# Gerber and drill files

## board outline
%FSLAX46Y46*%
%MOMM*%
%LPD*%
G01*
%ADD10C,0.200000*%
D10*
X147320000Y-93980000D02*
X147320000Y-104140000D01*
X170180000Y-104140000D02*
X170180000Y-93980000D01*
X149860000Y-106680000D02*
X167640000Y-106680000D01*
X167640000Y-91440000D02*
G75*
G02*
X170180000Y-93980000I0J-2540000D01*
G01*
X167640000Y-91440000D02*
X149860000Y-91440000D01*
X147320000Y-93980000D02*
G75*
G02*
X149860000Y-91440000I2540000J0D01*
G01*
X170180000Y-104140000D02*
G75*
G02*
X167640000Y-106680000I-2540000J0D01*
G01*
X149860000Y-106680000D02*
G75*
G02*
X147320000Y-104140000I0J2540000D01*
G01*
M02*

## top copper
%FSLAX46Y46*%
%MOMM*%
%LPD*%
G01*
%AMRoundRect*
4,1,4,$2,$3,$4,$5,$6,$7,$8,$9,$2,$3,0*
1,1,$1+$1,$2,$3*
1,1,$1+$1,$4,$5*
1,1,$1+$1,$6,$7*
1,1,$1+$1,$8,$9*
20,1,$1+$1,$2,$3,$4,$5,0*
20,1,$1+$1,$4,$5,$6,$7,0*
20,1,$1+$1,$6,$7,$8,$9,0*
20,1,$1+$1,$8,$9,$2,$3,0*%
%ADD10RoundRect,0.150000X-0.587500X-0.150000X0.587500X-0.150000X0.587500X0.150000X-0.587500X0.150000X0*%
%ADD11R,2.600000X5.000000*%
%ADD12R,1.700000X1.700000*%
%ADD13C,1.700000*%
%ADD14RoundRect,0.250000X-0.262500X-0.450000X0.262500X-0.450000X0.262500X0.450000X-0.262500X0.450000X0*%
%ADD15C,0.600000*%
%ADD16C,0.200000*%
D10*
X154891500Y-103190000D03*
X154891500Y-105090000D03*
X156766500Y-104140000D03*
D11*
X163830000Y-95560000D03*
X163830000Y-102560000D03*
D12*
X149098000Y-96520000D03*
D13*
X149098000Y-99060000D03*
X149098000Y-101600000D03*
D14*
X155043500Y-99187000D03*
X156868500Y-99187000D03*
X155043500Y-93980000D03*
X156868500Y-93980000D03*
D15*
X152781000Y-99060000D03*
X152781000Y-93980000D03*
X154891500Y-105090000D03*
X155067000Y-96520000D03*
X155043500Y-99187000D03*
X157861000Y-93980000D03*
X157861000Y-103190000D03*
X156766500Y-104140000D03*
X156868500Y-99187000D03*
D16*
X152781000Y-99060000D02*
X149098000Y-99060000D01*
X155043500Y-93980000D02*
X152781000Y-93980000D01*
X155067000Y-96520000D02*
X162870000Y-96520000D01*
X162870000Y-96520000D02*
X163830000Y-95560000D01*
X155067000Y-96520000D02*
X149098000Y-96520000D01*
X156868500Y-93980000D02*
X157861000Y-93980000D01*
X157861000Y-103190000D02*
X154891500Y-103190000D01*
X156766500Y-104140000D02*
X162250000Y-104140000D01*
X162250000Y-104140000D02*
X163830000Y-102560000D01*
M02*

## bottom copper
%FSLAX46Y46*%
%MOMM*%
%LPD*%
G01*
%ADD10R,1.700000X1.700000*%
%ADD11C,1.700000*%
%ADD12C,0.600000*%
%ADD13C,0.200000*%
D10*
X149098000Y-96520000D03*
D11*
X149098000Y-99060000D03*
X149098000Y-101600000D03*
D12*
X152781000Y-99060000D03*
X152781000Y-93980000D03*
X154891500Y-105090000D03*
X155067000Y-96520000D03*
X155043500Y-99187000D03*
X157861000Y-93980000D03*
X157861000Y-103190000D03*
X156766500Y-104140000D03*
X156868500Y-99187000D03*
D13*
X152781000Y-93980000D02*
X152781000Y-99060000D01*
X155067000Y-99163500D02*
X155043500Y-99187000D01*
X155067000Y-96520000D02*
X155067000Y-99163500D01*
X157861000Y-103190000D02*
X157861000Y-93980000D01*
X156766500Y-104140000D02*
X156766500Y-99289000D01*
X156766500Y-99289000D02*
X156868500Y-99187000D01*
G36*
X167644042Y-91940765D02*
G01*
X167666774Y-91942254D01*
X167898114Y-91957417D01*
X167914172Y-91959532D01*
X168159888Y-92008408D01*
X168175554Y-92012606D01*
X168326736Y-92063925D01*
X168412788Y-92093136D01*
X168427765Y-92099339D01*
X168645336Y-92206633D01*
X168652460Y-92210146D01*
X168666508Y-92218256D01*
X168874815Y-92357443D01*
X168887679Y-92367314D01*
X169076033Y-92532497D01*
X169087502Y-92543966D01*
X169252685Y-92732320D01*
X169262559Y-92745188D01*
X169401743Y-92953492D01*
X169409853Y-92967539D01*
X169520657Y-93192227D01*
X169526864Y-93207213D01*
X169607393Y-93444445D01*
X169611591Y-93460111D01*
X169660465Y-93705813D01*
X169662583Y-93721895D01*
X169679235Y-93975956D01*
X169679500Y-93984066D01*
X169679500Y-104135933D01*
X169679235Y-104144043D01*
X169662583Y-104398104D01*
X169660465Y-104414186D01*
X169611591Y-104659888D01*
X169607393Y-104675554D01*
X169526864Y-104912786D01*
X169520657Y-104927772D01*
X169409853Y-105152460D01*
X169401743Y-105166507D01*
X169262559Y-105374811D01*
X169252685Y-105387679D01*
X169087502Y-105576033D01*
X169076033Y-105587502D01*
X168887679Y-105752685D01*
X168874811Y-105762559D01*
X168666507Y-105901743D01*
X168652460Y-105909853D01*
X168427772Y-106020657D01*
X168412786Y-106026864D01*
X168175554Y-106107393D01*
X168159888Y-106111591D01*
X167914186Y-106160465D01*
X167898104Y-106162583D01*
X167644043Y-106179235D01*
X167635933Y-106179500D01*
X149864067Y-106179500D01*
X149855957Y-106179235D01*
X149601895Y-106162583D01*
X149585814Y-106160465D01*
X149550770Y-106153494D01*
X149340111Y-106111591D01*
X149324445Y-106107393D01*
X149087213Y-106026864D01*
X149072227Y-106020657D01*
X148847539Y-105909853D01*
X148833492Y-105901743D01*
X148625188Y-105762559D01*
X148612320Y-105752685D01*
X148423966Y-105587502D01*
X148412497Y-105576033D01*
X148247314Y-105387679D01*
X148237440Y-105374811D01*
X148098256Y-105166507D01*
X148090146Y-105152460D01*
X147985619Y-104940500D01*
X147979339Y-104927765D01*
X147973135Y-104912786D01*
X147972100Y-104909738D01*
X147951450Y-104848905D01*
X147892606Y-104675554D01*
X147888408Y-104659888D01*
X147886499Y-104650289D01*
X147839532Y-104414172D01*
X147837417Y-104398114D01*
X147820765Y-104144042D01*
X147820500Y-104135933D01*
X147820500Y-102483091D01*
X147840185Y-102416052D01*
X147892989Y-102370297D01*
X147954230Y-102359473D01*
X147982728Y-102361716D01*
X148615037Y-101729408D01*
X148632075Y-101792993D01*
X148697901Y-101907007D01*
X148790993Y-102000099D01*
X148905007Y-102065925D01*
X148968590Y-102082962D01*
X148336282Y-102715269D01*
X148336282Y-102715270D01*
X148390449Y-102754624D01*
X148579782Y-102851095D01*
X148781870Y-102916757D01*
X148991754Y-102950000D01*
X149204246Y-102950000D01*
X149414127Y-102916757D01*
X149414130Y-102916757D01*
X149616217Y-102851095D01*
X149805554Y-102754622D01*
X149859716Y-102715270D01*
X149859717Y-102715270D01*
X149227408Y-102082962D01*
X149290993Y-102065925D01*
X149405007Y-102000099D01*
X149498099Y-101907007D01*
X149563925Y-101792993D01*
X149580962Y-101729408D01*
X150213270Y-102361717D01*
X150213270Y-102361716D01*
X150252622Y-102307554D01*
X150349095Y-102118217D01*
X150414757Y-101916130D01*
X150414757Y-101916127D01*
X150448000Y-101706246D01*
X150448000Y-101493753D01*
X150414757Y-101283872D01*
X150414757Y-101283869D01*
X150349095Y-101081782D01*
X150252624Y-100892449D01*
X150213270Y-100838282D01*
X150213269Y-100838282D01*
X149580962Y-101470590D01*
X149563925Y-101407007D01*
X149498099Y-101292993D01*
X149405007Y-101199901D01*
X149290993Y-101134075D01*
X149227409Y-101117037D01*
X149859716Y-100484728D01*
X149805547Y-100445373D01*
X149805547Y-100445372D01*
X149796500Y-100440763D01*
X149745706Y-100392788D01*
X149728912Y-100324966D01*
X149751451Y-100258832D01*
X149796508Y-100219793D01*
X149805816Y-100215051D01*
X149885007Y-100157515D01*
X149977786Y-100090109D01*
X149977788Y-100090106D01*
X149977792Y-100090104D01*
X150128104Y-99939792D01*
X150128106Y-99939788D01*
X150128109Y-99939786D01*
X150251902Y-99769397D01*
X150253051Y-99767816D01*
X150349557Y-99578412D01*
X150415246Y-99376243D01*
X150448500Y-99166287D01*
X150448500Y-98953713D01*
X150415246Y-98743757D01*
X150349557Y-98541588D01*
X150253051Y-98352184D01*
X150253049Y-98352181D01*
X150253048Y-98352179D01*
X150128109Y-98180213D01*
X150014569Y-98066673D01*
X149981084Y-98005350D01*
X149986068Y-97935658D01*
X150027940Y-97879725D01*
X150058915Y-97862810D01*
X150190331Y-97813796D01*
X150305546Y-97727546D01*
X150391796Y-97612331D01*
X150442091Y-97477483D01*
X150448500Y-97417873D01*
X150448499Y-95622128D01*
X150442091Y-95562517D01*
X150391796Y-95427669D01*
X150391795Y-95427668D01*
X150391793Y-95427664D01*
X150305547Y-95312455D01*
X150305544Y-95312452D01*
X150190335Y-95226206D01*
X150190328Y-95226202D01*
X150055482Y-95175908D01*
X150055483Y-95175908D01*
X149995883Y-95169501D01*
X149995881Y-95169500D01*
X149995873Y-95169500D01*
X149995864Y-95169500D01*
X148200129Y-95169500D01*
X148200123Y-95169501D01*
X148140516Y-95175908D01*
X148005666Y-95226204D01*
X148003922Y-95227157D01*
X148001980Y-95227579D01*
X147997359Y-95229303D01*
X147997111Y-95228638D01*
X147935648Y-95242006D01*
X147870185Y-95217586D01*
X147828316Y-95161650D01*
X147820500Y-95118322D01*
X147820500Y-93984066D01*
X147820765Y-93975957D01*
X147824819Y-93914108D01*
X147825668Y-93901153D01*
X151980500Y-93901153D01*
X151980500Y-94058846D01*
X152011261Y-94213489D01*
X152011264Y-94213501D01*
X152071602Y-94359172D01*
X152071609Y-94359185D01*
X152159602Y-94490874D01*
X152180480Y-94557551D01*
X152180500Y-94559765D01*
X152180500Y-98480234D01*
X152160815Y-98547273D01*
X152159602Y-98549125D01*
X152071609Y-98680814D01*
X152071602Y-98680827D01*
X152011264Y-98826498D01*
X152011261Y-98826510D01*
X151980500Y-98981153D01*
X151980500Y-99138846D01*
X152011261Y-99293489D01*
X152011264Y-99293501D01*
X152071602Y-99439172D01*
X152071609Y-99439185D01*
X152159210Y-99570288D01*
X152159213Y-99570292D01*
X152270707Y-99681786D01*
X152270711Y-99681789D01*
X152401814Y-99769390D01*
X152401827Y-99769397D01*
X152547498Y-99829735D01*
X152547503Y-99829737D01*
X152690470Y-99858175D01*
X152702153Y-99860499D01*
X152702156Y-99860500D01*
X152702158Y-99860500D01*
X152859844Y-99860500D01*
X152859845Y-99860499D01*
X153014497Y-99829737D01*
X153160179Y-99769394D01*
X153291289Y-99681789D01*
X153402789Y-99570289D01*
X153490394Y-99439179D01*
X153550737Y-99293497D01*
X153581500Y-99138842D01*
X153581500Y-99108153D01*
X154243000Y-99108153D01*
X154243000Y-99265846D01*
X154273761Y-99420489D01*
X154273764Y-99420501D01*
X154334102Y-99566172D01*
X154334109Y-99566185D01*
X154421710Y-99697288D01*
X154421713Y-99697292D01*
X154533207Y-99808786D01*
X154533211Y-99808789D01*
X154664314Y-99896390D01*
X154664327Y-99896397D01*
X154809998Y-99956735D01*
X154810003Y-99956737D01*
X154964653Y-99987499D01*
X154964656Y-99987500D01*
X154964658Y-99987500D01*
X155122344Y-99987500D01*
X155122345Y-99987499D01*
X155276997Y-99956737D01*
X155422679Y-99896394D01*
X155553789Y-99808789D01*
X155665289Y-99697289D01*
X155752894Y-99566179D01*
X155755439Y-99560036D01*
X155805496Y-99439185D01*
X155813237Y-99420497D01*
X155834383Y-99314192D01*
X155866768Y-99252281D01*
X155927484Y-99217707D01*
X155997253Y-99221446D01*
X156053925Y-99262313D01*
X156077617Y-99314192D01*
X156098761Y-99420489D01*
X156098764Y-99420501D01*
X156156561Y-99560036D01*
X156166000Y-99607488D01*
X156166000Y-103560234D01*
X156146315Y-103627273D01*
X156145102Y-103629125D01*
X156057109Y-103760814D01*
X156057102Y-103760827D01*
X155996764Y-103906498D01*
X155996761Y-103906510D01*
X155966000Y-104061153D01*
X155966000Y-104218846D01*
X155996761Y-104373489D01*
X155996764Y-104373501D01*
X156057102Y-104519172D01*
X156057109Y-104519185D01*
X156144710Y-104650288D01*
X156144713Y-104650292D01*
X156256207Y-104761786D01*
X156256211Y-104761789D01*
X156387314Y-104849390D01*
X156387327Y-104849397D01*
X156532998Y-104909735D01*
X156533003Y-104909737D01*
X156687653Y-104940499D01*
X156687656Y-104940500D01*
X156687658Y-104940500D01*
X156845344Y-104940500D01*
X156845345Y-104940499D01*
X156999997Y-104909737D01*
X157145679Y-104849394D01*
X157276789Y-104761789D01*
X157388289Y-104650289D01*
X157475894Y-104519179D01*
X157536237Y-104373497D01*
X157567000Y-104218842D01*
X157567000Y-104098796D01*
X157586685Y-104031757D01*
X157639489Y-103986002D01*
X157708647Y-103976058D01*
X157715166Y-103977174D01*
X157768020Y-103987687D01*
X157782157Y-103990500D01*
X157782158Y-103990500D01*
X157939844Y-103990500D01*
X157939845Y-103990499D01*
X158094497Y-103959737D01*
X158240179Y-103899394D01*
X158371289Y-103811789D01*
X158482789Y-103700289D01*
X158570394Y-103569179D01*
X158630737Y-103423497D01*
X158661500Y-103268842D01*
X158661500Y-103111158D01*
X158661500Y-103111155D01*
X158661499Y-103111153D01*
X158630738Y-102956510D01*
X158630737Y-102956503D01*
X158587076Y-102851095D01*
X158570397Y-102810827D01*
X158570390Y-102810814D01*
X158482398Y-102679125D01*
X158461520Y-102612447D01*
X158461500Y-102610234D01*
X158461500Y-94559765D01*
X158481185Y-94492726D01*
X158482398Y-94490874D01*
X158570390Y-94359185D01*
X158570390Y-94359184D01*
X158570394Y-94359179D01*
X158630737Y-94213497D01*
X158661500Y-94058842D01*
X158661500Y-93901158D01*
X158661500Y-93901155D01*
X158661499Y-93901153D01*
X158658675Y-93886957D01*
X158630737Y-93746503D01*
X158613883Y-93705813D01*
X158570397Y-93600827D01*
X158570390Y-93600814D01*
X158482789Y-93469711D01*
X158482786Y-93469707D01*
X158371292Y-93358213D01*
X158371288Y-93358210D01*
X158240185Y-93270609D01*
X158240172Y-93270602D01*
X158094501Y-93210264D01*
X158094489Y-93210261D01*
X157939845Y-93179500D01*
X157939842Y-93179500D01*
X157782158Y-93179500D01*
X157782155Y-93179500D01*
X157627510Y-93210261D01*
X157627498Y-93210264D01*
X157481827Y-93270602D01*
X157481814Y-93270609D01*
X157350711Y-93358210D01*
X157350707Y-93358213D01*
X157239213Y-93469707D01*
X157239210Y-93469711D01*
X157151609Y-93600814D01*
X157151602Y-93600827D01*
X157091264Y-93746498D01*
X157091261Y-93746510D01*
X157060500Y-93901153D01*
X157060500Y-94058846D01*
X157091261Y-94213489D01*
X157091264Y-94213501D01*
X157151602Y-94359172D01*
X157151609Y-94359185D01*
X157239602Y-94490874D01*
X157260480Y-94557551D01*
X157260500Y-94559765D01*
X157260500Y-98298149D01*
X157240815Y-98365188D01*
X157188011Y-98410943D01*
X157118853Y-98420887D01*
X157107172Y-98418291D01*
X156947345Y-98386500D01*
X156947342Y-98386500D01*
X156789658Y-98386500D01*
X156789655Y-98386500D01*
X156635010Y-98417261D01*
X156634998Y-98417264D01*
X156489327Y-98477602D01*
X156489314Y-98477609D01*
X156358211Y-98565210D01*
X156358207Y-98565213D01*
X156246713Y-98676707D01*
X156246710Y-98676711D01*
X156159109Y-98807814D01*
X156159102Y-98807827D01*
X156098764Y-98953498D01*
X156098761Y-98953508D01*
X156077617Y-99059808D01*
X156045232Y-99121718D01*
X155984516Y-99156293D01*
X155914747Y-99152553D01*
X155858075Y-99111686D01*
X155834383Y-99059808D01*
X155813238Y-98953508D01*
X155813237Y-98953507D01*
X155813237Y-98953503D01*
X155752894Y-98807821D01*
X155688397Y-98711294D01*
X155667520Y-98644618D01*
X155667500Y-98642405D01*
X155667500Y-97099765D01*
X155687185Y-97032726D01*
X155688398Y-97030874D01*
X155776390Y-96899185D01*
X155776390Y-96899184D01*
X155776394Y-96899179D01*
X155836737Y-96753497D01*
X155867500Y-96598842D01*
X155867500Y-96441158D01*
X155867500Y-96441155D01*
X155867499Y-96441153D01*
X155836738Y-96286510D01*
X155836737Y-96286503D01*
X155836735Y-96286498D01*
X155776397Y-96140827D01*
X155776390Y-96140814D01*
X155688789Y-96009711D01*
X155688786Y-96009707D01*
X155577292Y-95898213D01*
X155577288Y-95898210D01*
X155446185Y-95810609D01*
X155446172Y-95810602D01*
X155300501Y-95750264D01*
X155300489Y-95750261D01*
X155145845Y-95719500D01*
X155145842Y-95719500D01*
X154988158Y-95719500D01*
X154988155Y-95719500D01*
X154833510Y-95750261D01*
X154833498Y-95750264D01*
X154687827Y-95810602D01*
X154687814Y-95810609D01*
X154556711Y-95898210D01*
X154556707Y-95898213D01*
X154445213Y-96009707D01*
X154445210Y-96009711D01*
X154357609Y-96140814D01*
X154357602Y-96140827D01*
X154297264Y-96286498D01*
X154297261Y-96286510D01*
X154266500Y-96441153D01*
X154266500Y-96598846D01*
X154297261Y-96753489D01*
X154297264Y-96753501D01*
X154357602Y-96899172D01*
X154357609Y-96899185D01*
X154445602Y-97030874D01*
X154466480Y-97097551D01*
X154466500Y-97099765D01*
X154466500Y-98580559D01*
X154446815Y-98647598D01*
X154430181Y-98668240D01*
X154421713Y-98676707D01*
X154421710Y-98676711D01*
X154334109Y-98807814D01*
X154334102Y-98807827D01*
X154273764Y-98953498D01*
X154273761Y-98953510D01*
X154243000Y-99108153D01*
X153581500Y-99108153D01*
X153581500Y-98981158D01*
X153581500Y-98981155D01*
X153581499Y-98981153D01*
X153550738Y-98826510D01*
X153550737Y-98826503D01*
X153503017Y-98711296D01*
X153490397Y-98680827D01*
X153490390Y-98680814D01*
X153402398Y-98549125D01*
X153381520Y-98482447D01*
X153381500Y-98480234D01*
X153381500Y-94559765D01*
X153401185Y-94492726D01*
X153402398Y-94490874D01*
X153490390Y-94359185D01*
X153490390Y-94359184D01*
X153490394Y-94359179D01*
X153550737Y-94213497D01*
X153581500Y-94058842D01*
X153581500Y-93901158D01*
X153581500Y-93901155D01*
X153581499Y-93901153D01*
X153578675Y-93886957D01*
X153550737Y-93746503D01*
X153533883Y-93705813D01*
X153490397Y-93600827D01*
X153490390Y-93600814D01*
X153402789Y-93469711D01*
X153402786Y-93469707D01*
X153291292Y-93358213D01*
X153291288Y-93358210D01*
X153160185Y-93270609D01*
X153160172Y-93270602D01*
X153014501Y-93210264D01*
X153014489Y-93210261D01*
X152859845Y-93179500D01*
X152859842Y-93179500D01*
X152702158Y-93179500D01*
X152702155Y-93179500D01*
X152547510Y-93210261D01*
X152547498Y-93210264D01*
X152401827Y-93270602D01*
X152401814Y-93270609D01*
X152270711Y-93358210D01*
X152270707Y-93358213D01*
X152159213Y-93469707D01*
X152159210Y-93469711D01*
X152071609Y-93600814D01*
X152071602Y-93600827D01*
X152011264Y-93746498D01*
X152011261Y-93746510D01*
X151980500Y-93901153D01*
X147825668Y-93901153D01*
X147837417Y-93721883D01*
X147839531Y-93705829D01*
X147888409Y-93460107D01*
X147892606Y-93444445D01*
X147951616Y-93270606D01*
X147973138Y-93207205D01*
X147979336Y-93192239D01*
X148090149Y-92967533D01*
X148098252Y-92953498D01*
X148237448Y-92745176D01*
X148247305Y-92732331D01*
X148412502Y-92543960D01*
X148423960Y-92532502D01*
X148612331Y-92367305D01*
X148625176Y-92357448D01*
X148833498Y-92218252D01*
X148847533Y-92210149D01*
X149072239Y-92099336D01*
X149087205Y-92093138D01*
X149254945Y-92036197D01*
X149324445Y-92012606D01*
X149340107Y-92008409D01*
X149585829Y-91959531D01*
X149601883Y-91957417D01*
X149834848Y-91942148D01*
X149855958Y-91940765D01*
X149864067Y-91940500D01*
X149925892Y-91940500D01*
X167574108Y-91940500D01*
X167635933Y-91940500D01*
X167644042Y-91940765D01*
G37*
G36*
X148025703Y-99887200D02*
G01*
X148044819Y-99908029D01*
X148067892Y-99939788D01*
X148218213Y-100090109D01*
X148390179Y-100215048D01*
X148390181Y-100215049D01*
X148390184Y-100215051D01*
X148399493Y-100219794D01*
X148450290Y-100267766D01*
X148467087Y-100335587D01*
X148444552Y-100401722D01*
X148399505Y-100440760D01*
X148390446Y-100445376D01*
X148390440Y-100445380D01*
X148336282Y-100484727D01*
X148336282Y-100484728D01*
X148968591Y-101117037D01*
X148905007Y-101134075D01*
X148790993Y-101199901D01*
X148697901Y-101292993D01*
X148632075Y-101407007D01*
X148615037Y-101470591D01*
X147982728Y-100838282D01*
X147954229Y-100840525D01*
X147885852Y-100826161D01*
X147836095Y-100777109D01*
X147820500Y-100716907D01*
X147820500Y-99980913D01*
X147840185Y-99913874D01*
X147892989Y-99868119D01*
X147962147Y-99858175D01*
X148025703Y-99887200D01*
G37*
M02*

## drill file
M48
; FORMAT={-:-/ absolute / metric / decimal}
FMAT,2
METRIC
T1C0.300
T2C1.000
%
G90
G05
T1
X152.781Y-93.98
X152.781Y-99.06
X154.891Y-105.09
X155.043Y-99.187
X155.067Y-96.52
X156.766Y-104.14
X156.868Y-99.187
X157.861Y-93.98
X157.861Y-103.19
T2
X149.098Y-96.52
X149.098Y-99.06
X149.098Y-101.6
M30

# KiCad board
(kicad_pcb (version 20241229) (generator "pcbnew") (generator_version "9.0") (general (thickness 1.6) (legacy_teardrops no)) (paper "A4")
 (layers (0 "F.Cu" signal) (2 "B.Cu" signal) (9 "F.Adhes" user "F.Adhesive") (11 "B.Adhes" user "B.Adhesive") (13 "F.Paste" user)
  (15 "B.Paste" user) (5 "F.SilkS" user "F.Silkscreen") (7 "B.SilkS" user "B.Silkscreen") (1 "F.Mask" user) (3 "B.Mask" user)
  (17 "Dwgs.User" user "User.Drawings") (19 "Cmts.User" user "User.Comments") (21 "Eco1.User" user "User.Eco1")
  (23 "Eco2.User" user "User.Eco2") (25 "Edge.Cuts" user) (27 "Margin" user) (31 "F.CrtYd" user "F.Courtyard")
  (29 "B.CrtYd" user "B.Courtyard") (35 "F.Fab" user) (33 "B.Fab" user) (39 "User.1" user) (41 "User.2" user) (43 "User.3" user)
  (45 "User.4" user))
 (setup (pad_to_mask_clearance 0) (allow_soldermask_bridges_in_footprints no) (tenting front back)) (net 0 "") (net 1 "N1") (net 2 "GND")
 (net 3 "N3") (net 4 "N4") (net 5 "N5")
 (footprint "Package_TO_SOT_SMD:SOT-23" (layer "F.Cu") (at 155.829 104.14)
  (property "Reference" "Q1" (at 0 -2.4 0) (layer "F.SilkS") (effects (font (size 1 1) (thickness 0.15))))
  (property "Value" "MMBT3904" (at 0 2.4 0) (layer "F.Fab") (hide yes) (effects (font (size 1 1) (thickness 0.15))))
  (pad "1" smd roundrect (at -0.9375 -0.95) (size 1.475 0.6) (layers "F.Cu" "F.Mask" "F.Paste") (roundrect_rratio 0.25) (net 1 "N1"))
  (pad "2" smd roundrect (at -0.9375 0.95) (size 1.475 0.6) (layers "F.Cu" "F.Mask" "F.Paste") (roundrect_rratio 0.25) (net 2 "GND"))
  (pad "3" smd roundrect (at 0.9375 0) (size 1.475 0.6) (layers "F.Cu" "F.Mask" "F.Paste") (roundrect_rratio 0.25) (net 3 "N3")))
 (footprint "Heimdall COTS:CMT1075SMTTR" (layer "F.Cu") (at 163.83 99.06 180)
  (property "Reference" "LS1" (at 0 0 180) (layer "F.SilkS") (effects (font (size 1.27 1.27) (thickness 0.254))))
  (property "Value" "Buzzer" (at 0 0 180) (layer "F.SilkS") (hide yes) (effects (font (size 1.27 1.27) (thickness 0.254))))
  (pad "1" smd rect (at 0 3.5 180) (size 2.6 5) (layers "F.Cu" "F.Mask" "F.Paste") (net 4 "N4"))
  (pad "2" smd rect (at 0 -3.5 180) (size 2.6 5) (layers "F.Cu" "F.Mask" "F.Paste") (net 3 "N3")))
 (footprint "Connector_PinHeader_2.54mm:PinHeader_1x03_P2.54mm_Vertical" (layer "F.Cu") (at 149.098 96.52)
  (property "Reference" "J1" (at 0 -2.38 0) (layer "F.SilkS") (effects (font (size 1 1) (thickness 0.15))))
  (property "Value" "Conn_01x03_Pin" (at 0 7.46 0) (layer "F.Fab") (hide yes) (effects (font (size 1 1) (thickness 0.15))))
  (pad "1" thru_hole rect (at 0 0) (size 1.7 1.7) (drill 1) (layers "*.Cu" "*.Mask") (remove_unused_layers no) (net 4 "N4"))
  (pad "2" thru_hole circle (at 0 2.54) (size 1.7 1.7) (drill 1) (layers "*.Cu" "*.Mask") (remove_unused_layers no) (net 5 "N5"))
  (pad "3" thru_hole circle (at 0 5.08) (size 1.7 1.7) (drill 1) (layers "*.Cu" "*.Mask") (remove_unused_layers no) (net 2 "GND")))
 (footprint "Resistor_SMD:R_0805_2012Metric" (layer "F.Cu") (at 155.956 99.187)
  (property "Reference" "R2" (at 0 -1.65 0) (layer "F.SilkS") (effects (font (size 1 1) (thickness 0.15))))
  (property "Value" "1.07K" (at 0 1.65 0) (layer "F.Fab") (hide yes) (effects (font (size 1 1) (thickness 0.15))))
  (pad "1" smd roundrect (at -0.9125 0) (size 1.025 1.4) (layers "F.Cu" "F.Mask" "F.Paste") (roundrect_rratio 0.243902) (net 4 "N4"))
  (pad "2" smd roundrect (at 0.9125 0) (size 1.025 1.4) (layers "F.Cu" "F.Mask" "F.Paste") (roundrect_rratio 0.243902) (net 3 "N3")))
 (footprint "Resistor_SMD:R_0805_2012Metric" (layer "F.Cu") (at 155.956 93.98)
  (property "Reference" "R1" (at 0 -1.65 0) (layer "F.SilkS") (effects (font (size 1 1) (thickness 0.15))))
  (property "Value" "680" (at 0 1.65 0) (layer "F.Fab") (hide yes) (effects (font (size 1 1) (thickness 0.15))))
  (pad "1" smd roundrect (at -0.9125 0) (size 1.025 1.4) (layers "F.Cu" "F.Mask" "F.Paste") (roundrect_rratio 0.243902) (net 5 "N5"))
  (pad "2" smd roundrect (at 0.9125 0) (size 1.025 1.4) (layers "F.Cu" "F.Mask" "F.Paste") (roundrect_rratio 0.243902) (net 1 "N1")))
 (gr_line (start 147.32 93.98) (end 147.32 104.14) (stroke (width 0.2) (type solid)) (layer "Edge.Cuts"))
 (gr_line (start 170.18 104.14) (end 170.18 93.98) (stroke (width 0.2) (type solid)) (layer "Edge.Cuts"))
 (gr_line (start 149.86 106.68) (end 167.64 106.68) (stroke (width 0.2) (type solid)) (layer "Edge.Cuts"))
 (gr_arc (start 167.64 91.44) (mid 169.436051 92.183949) (end 170.18 93.98) (stroke (width 0.2) (type solid)) (layer "Edge.Cuts"))
 (gr_line (start 167.64 91.44) (end 149.86 91.44) (stroke (width 0.2) (type solid)) (layer "Edge.Cuts"))
 (gr_arc (start 147.32 93.98) (mid 148.063949 92.183949) (end 149.86 91.44) (stroke (width 0.2) (type solid)) (layer "Edge.Cuts"))
 (gr_arc (start 170.18 104.14) (mid 169.436051 105.936051) (end 167.64 106.68) (stroke (width 0.2) (type solid)) (layer "Edge.Cuts"))
 (gr_arc (start 149.86 106.68) (mid 148.063949 105.936051) (end 147.32 104.14) (stroke (width 0.2) (type solid)) (layer "Edge.Cuts"))
 (segment (start 152.781 99.06) (end 149.098 99.06) (width 0.2) (layer "F.Cu") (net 5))
 (segment (start 155.0435 93.98) (end 152.781 93.98) (width 0.2) (layer "F.Cu") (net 5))
 (via (at 152.781 99.06) (size 0.6) (drill 0.3) (layers "F.Cu" "B.Cu") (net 5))
 (via (at 152.781 93.98) (size 0.6) (drill 0.3) (layers "F.Cu" "B.Cu") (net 5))
 (segment (start 152.781 93.98) (end 152.781 99.06) (width 0.2) (layer "B.Cu") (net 5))
 (via (at 154.8915 105.09) (size 0.6) (drill 0.3) (layers "F.Cu" "B.Cu") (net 2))
 (segment (start 155.067 96.52) (end 162.87 96.52) (width 0.2) (layer "F.Cu") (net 4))
 (segment (start 162.87 96.52) (end 163.83 95.56) (width 0.2) (layer "F.Cu") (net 4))
 (segment (start 155.067 96.52) (end 149.098 96.52) (width 0.2) (layer "F.Cu") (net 4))
 (via (at 155.067 96.52) (size 0.6) (drill 0.3) (layers "F.Cu" "B.Cu") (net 4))
 (via (at 155.0435 99.187) (size 0.6) (drill 0.3) (layers "F.Cu" "B.Cu") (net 4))
 (segment (start 155.067 99.1635) (end 155.0435 99.187) (width 0.2) (layer "B.Cu") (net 4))
 (segment (start 155.067 96.52) (end 155.067 99.1635) (width 0.2) (layer "B.Cu") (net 4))
 (segment (start 156.8685 93.98) (end 157.861 93.98) (width 0.2) (layer "F.Cu") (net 1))
 (segment (start 157.861 103.19) (end 154.8915 103.19) (width 0.2) (layer "F.Cu") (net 1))
 (via (at 157.861 93.98) (size 0.6) (drill 0.3) (layers "F.Cu" "B.Cu") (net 1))
 (via (at 157.861 103.19) (size 0.6) (drill 0.3) (layers "F.Cu" "B.Cu") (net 1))
 (segment (start 157.861 103.19) (end 157.861 93.98) (width 0.2) (layer "B.Cu") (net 1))
 (segment (start 156.7665 104.14) (end 162.25 104.14) (width 0.2) (layer "F.Cu") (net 3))
 (segment (start 162.25 104.14) (end 163.83 102.56) (width 0.2) (layer "F.Cu") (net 3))
 (via (at 156.7665 104.14) (size 0.6) (drill 0.3) (layers "F.Cu" "B.Cu") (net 3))
 (via (at 156.8685 99.187) (size 0.6) (drill 0.3) (layers "F.Cu" "B.Cu") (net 3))
 (segment (start 156.7665 104.14) (end 156.7665 99.289) (width 0.2) (layer "B.Cu") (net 3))
 (segment (start 156.7665 99.289) (end 156.8685 99.187) (width 0.2) (layer "B.Cu") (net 3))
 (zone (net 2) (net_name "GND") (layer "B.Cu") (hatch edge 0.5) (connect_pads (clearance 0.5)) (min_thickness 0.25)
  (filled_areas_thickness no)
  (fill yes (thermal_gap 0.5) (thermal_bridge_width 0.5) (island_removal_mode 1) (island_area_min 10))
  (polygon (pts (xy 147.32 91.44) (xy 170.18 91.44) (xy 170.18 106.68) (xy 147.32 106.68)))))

